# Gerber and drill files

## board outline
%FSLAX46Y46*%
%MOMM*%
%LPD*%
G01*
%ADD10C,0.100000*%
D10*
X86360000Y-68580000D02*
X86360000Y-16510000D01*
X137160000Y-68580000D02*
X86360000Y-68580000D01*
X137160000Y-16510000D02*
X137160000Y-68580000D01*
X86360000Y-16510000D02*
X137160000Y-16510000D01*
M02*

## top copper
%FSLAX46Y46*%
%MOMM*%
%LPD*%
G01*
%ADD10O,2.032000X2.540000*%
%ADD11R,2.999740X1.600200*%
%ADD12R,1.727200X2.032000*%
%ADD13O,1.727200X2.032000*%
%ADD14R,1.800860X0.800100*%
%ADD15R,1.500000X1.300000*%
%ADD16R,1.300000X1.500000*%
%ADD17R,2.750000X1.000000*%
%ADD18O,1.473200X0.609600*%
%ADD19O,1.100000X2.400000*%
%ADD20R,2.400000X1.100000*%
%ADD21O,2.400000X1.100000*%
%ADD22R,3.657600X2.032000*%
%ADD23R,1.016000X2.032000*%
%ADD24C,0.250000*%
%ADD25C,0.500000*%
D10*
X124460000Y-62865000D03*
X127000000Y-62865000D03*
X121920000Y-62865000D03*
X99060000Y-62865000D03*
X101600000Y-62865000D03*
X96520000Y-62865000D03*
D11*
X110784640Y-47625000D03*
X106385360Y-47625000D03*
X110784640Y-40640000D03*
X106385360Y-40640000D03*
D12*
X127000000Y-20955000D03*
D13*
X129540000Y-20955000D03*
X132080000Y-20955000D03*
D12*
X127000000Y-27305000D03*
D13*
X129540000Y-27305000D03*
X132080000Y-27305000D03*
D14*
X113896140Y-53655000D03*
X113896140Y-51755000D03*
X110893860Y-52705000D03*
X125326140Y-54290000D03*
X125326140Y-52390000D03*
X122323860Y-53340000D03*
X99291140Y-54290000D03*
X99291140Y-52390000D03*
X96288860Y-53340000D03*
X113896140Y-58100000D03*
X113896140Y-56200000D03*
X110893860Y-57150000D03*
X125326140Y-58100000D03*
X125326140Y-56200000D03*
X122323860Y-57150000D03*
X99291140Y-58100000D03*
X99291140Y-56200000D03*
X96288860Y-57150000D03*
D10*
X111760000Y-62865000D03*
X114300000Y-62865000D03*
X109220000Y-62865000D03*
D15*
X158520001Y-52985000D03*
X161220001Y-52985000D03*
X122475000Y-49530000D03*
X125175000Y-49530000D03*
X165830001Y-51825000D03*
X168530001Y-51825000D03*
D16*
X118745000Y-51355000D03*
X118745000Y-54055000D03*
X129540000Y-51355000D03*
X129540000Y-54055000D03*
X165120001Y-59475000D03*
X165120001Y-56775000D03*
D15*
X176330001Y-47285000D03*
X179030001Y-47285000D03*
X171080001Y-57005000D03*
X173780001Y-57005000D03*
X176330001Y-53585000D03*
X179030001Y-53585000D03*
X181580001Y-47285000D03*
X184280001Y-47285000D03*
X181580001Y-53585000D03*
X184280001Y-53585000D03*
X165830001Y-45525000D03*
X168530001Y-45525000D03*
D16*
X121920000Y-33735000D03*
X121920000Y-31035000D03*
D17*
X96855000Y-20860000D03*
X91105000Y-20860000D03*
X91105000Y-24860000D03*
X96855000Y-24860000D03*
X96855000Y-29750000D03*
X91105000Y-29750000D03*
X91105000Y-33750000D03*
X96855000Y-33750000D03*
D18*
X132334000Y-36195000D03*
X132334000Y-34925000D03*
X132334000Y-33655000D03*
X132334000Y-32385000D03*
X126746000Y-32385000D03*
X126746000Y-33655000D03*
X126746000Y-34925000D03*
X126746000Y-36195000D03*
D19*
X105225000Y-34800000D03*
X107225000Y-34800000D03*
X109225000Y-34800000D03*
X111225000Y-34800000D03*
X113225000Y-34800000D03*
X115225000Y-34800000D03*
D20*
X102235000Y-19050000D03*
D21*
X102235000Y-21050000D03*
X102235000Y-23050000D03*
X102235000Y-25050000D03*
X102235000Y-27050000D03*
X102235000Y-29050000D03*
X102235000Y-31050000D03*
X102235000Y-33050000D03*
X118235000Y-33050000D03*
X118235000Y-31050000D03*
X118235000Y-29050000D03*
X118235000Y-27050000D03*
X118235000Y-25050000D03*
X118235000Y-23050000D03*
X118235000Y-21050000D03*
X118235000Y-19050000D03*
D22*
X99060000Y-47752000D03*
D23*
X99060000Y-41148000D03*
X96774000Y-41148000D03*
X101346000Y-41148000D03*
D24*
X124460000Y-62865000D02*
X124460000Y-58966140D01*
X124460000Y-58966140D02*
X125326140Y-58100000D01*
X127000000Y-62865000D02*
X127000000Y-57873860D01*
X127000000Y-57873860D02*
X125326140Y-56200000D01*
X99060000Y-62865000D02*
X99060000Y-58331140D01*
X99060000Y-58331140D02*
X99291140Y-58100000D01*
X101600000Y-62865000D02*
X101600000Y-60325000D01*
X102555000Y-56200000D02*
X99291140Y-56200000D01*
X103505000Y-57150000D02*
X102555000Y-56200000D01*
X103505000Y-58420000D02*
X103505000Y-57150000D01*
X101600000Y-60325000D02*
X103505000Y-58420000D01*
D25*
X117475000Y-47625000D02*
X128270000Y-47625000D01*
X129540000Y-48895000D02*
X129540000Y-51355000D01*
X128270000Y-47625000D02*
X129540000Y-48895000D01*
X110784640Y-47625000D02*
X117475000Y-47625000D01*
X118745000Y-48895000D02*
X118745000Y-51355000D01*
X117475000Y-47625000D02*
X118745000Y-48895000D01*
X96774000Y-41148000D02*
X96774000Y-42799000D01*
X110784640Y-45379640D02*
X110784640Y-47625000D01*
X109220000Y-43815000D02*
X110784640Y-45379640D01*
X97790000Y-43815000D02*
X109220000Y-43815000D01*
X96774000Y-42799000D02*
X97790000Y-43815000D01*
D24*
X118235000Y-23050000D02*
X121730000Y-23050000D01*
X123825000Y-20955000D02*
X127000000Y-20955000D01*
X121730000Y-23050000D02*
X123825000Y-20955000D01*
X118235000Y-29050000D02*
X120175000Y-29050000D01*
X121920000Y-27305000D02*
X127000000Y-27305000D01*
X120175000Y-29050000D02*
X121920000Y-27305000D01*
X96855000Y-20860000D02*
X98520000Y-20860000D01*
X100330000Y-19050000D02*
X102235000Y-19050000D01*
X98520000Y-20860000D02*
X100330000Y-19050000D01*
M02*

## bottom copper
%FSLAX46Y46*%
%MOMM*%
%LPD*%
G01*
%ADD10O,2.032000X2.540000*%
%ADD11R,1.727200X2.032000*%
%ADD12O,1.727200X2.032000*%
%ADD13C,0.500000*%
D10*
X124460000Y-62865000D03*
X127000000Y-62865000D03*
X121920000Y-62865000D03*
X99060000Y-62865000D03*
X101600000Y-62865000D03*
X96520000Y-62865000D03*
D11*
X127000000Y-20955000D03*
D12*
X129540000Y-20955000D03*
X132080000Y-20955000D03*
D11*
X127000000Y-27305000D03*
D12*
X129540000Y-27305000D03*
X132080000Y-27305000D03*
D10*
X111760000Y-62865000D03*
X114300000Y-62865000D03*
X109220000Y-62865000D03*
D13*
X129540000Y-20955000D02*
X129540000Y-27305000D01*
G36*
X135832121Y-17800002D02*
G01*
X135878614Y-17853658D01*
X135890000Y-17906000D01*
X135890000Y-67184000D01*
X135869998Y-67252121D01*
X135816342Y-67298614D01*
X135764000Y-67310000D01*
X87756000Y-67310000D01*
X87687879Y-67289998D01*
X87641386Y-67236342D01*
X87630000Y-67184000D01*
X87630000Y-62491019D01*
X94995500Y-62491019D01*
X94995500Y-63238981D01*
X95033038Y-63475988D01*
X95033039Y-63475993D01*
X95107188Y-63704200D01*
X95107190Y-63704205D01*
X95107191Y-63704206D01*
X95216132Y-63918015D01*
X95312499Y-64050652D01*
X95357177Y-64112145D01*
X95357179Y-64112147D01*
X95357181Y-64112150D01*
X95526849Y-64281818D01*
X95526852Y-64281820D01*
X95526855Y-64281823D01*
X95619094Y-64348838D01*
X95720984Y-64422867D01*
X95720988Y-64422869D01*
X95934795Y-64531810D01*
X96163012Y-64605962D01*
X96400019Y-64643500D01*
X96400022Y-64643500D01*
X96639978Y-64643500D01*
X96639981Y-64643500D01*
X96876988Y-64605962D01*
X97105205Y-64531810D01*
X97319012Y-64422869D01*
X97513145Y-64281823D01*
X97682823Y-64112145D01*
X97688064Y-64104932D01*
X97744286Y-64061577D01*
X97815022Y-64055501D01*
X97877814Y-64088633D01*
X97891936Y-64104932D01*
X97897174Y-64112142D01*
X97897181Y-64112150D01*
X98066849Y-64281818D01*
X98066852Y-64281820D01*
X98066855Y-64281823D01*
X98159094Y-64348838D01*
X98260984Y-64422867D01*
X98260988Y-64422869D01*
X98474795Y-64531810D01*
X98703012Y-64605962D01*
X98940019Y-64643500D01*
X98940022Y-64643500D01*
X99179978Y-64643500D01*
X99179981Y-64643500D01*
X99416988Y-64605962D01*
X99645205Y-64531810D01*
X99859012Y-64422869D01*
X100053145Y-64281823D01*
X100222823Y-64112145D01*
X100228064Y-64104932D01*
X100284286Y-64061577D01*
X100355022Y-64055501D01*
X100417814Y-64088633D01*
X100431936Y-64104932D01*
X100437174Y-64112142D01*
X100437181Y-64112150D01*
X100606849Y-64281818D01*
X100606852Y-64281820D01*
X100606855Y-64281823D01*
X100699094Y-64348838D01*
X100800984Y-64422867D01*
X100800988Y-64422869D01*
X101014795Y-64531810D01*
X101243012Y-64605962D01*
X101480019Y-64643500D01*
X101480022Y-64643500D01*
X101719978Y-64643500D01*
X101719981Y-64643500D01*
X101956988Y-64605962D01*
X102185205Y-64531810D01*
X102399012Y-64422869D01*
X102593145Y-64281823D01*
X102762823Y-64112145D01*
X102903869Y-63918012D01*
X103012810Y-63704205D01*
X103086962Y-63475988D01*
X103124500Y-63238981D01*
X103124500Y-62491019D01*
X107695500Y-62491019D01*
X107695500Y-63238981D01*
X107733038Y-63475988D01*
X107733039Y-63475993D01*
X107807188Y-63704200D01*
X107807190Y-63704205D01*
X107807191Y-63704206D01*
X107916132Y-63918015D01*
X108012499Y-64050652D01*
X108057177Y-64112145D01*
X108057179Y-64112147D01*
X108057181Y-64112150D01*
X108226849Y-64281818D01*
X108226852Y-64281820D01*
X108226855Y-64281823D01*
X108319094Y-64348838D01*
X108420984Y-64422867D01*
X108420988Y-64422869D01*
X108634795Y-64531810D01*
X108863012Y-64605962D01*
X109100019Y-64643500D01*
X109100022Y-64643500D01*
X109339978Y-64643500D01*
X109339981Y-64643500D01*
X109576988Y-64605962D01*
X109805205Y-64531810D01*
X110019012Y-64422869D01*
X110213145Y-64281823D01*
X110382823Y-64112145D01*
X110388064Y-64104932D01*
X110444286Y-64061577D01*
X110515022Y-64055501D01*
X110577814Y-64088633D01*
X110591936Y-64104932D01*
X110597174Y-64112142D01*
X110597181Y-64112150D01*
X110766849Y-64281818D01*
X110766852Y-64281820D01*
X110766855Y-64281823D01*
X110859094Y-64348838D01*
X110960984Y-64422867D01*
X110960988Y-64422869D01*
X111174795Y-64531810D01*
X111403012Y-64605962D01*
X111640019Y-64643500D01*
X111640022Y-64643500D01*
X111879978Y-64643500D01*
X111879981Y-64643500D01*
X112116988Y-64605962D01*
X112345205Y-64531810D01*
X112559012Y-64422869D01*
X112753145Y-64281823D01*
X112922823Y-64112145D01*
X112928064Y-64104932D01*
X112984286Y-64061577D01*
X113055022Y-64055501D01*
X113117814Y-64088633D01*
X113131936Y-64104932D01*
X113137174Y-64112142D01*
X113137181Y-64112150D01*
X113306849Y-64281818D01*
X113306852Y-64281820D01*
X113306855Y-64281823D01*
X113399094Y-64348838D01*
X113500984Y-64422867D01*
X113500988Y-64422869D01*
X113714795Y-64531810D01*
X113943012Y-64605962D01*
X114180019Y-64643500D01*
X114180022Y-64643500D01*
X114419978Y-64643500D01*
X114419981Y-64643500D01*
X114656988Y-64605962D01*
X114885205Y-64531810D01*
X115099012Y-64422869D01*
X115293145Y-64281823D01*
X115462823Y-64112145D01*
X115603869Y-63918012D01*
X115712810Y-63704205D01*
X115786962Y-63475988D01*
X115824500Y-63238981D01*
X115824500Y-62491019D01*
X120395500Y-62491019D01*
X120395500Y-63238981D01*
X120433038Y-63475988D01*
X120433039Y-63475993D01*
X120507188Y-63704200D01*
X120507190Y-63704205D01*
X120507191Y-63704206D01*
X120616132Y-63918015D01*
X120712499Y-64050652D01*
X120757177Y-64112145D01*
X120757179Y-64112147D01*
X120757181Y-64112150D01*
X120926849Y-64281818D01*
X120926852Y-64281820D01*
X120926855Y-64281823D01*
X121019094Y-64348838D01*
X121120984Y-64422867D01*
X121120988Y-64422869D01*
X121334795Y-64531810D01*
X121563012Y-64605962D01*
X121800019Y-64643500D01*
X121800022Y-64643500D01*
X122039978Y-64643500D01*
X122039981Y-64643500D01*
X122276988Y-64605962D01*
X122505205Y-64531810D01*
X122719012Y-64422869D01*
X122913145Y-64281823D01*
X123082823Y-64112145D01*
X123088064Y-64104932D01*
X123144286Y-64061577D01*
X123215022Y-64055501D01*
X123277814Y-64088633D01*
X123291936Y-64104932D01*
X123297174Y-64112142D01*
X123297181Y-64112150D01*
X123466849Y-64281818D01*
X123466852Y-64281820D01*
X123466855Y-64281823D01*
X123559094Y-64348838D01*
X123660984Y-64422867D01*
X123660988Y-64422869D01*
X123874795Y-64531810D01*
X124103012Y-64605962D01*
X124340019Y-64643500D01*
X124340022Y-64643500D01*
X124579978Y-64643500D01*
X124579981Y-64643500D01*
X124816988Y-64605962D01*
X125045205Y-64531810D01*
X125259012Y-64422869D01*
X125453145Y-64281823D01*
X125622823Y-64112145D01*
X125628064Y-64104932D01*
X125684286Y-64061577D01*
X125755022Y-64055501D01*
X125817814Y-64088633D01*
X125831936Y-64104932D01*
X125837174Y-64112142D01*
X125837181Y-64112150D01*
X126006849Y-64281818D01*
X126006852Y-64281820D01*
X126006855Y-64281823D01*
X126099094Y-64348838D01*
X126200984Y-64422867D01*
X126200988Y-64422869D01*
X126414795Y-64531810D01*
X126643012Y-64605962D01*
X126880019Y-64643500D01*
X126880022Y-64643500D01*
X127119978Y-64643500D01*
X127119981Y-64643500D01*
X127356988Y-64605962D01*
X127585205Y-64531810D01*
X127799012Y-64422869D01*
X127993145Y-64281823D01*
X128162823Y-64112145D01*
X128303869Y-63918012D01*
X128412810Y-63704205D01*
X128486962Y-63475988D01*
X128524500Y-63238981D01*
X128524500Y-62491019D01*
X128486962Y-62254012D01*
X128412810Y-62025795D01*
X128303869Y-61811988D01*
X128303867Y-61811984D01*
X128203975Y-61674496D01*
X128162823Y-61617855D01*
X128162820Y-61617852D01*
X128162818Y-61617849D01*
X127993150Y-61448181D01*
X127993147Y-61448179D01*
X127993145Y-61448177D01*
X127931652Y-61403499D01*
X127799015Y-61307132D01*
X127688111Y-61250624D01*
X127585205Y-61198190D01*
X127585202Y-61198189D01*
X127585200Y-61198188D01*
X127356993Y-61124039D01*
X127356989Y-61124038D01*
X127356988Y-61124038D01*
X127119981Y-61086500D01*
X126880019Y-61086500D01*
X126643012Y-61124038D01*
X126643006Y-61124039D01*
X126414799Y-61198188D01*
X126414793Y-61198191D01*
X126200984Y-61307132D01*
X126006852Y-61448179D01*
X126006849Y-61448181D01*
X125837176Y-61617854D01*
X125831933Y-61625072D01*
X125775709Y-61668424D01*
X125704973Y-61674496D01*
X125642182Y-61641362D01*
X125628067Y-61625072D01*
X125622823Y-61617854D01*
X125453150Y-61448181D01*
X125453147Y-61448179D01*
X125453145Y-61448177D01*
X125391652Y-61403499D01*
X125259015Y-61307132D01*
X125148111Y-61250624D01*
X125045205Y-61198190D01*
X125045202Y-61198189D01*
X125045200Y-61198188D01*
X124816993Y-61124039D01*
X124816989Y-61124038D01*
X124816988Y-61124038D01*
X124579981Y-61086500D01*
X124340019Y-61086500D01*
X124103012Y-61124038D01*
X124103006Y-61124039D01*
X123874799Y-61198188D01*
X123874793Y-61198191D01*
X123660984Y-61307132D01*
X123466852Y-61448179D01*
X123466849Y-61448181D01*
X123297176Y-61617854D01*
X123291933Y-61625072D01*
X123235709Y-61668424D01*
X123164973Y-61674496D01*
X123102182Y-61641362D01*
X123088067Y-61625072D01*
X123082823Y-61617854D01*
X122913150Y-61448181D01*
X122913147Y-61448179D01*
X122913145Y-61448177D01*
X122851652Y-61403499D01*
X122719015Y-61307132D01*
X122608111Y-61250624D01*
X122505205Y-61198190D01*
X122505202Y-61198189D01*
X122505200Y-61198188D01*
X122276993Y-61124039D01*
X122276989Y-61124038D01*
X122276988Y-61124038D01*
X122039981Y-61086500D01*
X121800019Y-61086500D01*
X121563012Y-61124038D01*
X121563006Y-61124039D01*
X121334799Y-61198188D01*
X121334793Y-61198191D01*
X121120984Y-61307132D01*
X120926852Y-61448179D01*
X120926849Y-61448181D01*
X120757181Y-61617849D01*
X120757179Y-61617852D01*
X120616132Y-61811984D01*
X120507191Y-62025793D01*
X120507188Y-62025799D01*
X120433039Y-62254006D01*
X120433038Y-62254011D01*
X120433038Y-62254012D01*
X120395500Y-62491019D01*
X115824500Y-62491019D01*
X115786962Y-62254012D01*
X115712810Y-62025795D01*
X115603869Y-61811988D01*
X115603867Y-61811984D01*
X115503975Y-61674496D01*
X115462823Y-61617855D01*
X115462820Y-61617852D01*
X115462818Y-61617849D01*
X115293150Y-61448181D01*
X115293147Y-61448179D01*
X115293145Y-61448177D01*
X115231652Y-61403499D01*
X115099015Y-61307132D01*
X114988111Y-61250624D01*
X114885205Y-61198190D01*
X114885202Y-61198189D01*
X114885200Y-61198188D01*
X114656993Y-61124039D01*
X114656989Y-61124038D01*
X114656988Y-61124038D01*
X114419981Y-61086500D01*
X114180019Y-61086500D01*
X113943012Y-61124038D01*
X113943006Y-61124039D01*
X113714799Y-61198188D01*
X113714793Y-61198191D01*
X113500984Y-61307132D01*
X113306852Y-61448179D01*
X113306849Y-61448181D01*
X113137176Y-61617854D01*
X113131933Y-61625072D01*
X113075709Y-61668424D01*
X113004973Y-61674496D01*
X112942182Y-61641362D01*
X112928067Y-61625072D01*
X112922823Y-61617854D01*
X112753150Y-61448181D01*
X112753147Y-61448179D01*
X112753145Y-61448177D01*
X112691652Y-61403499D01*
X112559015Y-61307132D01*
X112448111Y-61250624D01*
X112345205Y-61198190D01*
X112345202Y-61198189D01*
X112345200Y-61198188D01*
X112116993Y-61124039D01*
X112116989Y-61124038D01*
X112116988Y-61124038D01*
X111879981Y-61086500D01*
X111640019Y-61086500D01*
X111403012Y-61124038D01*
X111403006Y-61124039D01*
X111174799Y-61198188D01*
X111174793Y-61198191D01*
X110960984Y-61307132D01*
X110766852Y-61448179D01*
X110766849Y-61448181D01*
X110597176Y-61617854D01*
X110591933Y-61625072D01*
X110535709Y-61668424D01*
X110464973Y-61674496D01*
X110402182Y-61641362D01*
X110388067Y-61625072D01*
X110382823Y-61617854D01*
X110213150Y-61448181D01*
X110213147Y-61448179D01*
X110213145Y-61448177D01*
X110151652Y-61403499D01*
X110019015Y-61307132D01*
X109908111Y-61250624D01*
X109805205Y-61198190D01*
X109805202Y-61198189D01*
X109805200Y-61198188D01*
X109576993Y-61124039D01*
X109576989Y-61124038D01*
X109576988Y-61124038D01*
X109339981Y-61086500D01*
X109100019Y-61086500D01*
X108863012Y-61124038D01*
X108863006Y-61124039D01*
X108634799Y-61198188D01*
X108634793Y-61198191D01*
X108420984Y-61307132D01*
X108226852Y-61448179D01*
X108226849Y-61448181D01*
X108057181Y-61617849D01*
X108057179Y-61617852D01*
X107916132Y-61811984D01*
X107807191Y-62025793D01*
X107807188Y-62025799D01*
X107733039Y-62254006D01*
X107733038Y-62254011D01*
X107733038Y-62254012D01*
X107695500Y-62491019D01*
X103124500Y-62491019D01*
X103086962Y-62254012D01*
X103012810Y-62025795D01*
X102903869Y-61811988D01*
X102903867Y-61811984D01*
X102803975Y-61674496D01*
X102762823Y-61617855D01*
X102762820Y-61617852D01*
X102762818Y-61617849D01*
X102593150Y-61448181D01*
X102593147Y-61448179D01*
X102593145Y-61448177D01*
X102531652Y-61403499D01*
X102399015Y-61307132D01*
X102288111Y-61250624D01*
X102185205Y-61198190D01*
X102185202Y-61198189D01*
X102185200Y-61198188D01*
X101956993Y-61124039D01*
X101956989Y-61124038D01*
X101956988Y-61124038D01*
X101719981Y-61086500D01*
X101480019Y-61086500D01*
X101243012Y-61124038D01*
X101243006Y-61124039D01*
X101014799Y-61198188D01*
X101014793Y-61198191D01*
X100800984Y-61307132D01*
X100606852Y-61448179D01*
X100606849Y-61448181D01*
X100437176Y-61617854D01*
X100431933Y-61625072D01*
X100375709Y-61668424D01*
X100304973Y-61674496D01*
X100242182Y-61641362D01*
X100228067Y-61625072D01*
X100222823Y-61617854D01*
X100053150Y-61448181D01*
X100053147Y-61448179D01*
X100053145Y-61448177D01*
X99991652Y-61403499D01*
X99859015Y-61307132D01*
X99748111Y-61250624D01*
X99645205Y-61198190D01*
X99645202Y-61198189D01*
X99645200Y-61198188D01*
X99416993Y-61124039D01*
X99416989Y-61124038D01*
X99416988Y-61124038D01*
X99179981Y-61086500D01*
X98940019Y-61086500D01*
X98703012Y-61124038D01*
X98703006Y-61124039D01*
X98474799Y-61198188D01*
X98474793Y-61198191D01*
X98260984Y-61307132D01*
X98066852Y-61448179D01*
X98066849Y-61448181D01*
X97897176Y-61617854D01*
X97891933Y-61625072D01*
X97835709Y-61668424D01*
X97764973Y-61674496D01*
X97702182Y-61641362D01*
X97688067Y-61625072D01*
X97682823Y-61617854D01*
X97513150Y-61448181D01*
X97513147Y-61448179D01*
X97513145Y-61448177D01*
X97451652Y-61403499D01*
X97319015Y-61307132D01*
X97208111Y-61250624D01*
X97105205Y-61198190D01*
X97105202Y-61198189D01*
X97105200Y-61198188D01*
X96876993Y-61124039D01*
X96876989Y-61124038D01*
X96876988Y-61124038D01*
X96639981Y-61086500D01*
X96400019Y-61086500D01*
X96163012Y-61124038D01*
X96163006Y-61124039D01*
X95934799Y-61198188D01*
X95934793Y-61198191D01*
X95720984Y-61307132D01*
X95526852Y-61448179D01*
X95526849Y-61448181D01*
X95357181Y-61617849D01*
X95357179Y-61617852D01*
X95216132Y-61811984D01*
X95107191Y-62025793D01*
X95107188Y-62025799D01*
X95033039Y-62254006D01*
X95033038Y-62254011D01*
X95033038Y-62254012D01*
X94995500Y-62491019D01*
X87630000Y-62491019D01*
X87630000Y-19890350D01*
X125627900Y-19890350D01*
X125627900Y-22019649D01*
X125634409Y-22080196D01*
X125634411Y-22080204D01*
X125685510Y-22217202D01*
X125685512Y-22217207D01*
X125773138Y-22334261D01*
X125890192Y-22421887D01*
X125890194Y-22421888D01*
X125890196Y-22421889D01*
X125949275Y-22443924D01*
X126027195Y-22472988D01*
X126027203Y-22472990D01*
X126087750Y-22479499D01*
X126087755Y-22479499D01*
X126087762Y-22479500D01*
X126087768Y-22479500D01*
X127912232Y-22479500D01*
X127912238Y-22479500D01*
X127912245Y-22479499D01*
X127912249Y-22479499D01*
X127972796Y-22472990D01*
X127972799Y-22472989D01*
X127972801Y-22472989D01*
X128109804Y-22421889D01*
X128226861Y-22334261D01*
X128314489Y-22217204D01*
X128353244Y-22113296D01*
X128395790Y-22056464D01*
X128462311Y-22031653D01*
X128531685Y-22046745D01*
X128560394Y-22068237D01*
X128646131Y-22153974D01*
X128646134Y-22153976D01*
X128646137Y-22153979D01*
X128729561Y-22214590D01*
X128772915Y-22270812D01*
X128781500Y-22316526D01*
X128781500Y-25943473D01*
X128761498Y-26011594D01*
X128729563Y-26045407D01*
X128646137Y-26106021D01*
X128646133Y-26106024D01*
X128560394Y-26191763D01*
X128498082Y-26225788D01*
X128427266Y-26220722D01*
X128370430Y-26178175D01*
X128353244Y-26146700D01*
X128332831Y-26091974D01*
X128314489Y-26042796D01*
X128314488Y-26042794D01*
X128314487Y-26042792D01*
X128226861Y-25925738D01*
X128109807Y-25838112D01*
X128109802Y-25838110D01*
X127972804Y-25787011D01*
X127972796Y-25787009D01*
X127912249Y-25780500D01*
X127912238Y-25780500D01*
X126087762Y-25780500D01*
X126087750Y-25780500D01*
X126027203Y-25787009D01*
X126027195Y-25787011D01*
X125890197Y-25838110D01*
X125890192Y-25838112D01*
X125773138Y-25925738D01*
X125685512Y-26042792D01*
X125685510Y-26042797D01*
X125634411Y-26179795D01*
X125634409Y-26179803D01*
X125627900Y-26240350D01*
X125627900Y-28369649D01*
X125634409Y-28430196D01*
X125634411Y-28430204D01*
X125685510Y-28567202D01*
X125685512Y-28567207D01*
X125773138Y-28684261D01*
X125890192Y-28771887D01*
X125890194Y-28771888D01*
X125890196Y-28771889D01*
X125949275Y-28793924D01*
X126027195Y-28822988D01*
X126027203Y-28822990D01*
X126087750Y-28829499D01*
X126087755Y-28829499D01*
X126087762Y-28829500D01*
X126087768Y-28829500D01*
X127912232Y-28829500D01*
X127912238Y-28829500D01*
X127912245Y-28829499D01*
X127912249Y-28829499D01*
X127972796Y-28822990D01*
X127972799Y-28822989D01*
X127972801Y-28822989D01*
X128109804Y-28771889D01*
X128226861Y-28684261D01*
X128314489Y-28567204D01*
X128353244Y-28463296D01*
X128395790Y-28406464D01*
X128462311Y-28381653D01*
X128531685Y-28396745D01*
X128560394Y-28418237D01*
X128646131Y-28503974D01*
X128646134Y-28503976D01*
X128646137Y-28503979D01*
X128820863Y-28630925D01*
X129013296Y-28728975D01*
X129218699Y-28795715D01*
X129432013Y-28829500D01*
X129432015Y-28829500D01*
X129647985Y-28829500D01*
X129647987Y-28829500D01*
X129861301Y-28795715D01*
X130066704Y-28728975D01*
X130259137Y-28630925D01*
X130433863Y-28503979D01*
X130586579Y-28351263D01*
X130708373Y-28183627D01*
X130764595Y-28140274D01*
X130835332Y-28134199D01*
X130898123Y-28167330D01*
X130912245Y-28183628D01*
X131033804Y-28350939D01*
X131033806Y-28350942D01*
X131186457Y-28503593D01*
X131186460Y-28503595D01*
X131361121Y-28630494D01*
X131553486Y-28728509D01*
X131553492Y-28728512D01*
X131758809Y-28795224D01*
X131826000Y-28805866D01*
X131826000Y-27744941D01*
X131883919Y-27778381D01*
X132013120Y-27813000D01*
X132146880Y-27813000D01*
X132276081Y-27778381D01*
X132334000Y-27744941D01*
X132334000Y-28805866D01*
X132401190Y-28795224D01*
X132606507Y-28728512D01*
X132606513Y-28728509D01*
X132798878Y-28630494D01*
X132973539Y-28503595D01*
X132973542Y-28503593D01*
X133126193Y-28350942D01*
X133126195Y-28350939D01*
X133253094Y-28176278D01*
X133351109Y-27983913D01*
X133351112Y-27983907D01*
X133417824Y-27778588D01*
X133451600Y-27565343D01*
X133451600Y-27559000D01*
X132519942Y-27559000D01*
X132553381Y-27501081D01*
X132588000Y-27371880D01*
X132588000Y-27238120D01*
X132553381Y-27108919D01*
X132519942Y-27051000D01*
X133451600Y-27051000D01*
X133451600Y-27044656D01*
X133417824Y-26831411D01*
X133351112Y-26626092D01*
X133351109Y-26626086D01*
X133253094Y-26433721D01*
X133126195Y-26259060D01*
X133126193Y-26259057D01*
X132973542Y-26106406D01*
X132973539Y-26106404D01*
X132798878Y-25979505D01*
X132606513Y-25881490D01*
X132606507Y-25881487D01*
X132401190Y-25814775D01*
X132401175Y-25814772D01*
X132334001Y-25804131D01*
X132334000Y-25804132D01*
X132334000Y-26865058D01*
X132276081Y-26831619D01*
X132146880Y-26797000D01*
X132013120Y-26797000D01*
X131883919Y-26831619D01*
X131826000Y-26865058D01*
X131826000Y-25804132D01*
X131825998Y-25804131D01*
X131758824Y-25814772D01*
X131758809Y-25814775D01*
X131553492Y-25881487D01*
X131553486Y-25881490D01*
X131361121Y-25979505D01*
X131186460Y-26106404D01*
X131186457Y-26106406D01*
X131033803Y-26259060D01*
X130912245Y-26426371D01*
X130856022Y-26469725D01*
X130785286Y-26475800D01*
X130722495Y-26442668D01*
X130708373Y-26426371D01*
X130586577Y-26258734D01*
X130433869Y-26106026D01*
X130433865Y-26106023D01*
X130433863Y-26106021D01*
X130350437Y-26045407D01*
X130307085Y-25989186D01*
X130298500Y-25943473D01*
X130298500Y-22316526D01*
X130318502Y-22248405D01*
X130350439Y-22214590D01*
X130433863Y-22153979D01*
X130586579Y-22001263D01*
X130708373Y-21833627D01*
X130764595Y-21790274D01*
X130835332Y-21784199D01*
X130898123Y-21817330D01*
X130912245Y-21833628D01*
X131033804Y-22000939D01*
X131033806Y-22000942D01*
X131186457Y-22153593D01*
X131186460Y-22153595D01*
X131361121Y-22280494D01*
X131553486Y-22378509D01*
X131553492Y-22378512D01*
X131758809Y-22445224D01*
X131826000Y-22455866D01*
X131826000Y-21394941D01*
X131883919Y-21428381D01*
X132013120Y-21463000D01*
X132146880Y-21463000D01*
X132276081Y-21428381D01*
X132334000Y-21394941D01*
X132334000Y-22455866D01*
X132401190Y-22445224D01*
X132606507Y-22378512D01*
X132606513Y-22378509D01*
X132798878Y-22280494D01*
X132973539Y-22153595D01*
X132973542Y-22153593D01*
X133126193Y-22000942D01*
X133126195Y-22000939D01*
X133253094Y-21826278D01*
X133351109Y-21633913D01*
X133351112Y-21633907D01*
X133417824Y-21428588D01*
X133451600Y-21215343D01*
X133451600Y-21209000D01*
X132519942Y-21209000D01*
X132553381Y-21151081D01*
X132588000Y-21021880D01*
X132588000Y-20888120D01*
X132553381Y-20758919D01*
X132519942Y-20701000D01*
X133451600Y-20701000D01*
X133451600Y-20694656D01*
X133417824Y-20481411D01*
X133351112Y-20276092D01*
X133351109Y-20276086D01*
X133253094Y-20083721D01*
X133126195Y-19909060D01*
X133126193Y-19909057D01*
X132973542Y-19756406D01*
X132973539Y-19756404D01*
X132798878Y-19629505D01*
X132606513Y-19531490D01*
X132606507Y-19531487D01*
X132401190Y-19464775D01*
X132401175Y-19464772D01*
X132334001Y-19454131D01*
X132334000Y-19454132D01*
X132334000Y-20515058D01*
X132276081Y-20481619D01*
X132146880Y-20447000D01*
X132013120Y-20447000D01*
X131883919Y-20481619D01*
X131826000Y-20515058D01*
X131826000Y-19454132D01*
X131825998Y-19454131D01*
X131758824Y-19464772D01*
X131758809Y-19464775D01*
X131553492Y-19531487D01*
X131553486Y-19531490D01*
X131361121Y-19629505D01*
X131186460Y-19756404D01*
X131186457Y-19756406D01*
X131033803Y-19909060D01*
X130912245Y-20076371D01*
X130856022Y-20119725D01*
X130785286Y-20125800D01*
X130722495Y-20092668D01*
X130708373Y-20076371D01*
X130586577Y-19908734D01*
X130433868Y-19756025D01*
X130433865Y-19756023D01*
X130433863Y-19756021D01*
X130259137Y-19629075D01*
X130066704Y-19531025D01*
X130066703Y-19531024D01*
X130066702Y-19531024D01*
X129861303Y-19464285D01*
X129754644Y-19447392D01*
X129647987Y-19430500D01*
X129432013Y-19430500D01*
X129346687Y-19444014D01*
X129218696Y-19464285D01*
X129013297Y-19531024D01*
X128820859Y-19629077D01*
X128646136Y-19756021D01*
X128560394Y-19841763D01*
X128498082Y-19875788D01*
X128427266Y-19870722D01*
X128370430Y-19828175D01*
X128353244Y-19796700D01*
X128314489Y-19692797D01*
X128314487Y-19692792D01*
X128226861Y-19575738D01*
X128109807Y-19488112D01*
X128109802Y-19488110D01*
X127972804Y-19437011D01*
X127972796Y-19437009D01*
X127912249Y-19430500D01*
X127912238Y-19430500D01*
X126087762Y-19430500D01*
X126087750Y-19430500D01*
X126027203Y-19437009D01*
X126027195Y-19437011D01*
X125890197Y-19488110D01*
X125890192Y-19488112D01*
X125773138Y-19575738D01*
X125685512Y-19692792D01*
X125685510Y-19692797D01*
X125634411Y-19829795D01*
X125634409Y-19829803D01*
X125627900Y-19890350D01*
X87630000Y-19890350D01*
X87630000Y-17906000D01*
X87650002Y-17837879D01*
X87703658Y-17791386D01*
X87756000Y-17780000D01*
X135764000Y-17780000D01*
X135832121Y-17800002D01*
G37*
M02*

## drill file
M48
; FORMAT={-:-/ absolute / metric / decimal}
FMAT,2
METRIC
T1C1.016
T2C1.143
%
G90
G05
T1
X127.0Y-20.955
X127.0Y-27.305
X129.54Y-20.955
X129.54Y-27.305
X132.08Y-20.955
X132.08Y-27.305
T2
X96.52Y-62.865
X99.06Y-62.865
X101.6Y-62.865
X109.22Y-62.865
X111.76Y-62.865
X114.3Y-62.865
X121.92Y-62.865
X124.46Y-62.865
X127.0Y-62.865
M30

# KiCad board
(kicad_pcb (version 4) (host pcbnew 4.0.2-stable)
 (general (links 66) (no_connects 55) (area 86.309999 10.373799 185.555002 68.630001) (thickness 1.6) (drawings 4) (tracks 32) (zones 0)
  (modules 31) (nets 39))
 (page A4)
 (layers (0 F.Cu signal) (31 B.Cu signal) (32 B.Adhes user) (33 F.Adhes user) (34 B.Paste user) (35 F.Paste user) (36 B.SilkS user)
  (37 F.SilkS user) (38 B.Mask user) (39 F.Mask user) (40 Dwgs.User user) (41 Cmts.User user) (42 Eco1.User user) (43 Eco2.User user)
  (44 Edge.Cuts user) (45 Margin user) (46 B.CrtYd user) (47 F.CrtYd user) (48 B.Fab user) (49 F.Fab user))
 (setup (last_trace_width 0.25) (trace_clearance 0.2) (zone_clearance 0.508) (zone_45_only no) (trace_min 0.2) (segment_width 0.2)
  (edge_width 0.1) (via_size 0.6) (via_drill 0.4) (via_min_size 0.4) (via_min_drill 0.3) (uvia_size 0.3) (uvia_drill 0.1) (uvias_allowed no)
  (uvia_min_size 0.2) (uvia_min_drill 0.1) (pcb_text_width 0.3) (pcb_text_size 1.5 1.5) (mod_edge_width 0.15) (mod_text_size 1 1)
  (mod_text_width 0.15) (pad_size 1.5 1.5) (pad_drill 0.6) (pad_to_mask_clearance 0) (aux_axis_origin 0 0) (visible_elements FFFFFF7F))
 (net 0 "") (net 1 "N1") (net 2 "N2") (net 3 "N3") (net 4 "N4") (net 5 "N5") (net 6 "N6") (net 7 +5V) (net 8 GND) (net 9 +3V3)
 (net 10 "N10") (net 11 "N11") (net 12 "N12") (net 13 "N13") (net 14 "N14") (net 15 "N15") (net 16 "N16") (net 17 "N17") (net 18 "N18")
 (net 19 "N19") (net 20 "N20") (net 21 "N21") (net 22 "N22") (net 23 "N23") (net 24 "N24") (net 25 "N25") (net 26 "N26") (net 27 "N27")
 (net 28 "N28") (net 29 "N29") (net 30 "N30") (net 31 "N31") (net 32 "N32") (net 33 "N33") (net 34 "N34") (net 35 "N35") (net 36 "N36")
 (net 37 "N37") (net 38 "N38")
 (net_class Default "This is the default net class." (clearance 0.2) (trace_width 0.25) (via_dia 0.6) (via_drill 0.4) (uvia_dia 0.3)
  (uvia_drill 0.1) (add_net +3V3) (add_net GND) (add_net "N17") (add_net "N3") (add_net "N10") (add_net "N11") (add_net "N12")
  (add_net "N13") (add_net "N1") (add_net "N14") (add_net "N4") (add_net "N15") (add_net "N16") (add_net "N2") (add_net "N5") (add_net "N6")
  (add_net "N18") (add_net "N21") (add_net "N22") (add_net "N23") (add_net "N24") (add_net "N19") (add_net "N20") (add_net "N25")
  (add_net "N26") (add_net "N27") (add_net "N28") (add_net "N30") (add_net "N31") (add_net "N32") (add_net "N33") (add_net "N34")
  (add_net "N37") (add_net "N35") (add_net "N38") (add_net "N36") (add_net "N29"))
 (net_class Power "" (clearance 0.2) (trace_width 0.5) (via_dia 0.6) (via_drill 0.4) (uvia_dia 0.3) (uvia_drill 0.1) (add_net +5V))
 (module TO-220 (layer F.Cu) (at 124.46 62.865)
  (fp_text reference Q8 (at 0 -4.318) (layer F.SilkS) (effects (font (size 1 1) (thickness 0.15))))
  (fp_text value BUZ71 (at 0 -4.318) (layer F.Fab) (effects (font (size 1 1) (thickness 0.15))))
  (pad 2 thru_hole oval (at 0 0) (size 2.032 2.54) (drill 1.143) (layers *.Cu *.Mask F.SilkS) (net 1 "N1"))
  (pad 3 thru_hole oval (at 2.54 0) (size 2.032 2.54) (drill 1.143) (layers *.Cu *.Mask F.SilkS) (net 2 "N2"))
  (pad 1 thru_hole oval (at -2.54 0) (size 2.032 2.54) (drill 1.143) (layers *.Cu *.Mask F.SilkS) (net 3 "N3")))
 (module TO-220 (layer F.Cu) (at 99.06 62.865)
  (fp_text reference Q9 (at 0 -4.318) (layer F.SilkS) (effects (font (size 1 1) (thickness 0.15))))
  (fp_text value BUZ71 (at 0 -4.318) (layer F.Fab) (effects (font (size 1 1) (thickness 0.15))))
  (pad 2 thru_hole oval (at 0 0) (size 2.032 2.54) (drill 1.143) (layers *.Cu *.Mask F.SilkS) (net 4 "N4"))
  (pad 3 thru_hole oval (at 2.54 0) (size 2.032 2.54) (drill 1.143) (layers *.Cu *.Mask F.SilkS) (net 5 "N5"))
  (pad 1 thru_hole oval (at -2.54 0) (size 2.032 2.54) (drill 1.143) (layers *.Cu *.Mask F.SilkS) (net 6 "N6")))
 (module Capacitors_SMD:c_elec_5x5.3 (layer F.Cu) (at 108.585 47.625)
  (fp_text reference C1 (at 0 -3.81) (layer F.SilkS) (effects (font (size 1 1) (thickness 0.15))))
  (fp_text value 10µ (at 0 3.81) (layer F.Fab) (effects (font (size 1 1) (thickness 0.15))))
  (pad 1 smd rect (at 2.19964 0) (size 2.99974 1.6002) (layers F.Cu F.Paste F.Mask) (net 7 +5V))
  (pad 2 smd rect (at -2.19964 0) (size 2.99974 1.6002) (layers F.Cu F.Paste F.Mask) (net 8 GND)))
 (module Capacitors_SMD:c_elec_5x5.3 (layer F.Cu) (at 108.585 40.64)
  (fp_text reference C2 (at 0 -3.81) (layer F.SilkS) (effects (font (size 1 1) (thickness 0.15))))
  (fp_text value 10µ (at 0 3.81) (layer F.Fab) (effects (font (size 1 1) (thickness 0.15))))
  (pad 1 smd rect (at 2.19964 0) (size 2.99974 1.6002) (layers F.Cu F.Paste F.Mask) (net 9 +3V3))
  (pad 2 smd rect (at -2.19964 0) (size 2.99974 1.6002) (layers F.Cu F.Paste F.Mask) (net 8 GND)))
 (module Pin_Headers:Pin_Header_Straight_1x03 (layer F.Cu) (at 127 20.955 90)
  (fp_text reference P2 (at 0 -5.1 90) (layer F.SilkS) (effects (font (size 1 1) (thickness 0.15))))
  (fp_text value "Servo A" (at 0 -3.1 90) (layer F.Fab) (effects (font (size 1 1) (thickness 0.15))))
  (pad 1 thru_hole rect (at 0 0 90) (size 2.032 1.7272) (drill 1.016) (layers *.Cu *.Mask F.SilkS) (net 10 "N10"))
  (pad 2 thru_hole oval (at 0 2.54 90) (size 2.032 1.7272) (drill 1.016) (layers *.Cu *.Mask F.SilkS) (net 7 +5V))
  (pad 3 thru_hole oval (at 0 5.08 90) (size 2.032 1.7272) (drill 1.016) (layers *.Cu *.Mask F.SilkS) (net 8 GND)))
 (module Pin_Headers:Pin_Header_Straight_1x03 (layer F.Cu) (at 127 27.305 90)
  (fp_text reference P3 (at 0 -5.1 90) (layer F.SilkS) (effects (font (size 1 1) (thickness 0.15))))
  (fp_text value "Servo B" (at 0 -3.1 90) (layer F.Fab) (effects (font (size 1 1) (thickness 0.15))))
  (pad 1 thru_hole rect (at 0 0 90) (size 2.032 1.7272) (drill 1.016) (layers *.Cu *.Mask F.SilkS) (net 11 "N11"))
  (pad 2 thru_hole oval (at 0 2.54 90) (size 2.032 1.7272) (drill 1.016) (layers *.Cu *.Mask F.SilkS) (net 7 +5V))
  (pad 3 thru_hole oval (at 0 5.08 90) (size 2.032 1.7272) (drill 1.016) (layers *.Cu *.Mask F.SilkS) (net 8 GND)))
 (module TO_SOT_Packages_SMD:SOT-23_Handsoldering (layer F.Cu) (at 112.395 52.705 90)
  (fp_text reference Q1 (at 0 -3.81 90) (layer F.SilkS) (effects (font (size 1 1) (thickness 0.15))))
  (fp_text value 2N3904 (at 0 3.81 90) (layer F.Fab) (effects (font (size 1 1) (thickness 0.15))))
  (pad 1 smd rect (at -0.95 1.50114 90) (size 0.8001 1.80086) (layers F.Cu F.Paste F.Mask) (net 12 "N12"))
  (pad 2 smd rect (at 0.95 1.50114 90) (size 0.8001 1.80086) (layers F.Cu F.Paste F.Mask) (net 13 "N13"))
  (pad 3 smd rect (at 0 -1.50114 90) (size 0.8001 1.80086) (layers F.Cu F.Paste F.Mask) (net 8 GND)))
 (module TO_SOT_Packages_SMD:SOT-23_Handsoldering (layer F.Cu) (at 123.825 53.34 90)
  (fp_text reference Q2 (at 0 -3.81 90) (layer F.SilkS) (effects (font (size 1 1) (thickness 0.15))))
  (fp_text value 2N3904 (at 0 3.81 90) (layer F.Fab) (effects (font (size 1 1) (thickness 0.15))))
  (pad 1 smd rect (at -0.95 1.50114 90) (size 0.8001 1.80086) (layers F.Cu F.Paste F.Mask) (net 1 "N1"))
  (pad 2 smd rect (at 0.95 1.50114 90) (size 0.8001 1.80086) (layers F.Cu F.Paste F.Mask) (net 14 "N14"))
  (pad 3 smd rect (at 0 -1.50114 90) (size 0.8001 1.80086) (layers F.Cu F.Paste F.Mask) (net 8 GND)))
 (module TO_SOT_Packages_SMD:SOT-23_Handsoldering (layer F.Cu) (at 97.79 53.34 90)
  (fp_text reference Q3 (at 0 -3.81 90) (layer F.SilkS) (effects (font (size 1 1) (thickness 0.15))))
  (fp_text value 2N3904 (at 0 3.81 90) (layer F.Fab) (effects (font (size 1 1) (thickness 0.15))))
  (pad 1 smd rect (at -0.95 1.50114 90) (size 0.8001 1.80086) (layers F.Cu F.Paste F.Mask) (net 4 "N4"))
  (pad 2 smd rect (at 0.95 1.50114 90) (size 0.8001 1.80086) (layers F.Cu F.Paste F.Mask) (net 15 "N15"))
  (pad 3 smd rect (at 0 -1.50114 90) (size 0.8001 1.80086) (layers F.Cu F.Paste F.Mask) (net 8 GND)))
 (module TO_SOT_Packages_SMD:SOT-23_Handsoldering (layer F.Cu) (at 112.395 57.15 90)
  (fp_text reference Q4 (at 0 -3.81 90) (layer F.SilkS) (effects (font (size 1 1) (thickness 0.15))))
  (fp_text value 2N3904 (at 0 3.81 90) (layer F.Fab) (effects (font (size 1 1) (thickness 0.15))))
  (pad 1 smd rect (at -0.95 1.50114 90) (size 0.8001 1.80086) (layers F.Cu F.Paste F.Mask) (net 12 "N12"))
  (pad 2 smd rect (at 0.95 1.50114 90) (size 0.8001 1.80086) (layers F.Cu F.Paste F.Mask) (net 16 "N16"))
  (pad 3 smd rect (at 0 -1.50114 90) (size 0.8001 1.80086) (layers F.Cu F.Paste F.Mask) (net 8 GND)))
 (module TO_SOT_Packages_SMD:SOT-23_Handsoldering (layer F.Cu) (at 123.825 57.15 90)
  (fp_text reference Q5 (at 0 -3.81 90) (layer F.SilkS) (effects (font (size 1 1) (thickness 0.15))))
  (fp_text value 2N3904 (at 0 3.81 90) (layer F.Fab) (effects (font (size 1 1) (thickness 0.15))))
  (pad 1 smd rect (at -0.95 1.50114 90) (size 0.8001 1.80086) (layers F.Cu F.Paste F.Mask) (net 1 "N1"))
  (pad 2 smd rect (at 0.95 1.50114 90) (size 0.8001 1.80086) (layers F.Cu F.Paste F.Mask) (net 2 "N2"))
  (pad 3 smd rect (at 0 -1.50114 90) (size 0.8001 1.80086) (layers F.Cu F.Paste F.Mask) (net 8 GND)))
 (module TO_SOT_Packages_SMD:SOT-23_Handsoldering (layer F.Cu) (at 97.79 57.15 90)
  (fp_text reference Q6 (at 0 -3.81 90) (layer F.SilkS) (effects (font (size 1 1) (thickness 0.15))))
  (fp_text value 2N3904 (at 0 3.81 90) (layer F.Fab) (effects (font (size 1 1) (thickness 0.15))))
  (pad 1 smd rect (at -0.95 1.50114 90) (size 0.8001 1.80086) (layers F.Cu F.Paste F.Mask) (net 4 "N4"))
  (pad 2 smd rect (at 0.95 1.50114 90) (size 0.8001 1.80086) (layers F.Cu F.Paste F.Mask) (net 5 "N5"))
  (pad 3 smd rect (at 0 -1.50114 90) (size 0.8001 1.80086) (layers F.Cu F.Paste F.Mask) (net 8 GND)))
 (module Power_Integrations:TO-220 (layer F.Cu) (at 111.76 62.865)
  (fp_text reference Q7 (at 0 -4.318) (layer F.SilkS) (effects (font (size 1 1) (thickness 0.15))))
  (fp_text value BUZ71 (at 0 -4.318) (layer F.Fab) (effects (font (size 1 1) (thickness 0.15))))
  (pad 2 thru_hole oval (at 0 0) (size 2.032 2.54) (drill 1.143) (layers *.Cu *.Mask F.SilkS) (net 12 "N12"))
  (pad 3 thru_hole oval (at 2.54 0) (size 2.032 2.54) (drill 1.143) (layers *.Cu *.Mask F.SilkS) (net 16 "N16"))
  (pad 1 thru_hole oval (at -2.54 0) (size 2.032 2.54) (drill 1.143) (layers *.Cu *.Mask F.SilkS) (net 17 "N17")))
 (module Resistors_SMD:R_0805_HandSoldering (layer F.Cu) (at 159.870001 52.985)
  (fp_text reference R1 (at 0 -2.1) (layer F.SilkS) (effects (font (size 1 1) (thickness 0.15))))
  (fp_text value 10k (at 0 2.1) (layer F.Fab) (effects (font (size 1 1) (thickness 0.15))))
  (pad 1 smd rect (at -1.35 0) (size 1.5 1.3) (layers F.Cu F.Paste F.Mask) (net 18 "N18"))
  (pad 2 smd rect (at 1.35 0) (size 1.5 1.3) (layers F.Cu F.Paste F.Mask) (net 13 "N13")))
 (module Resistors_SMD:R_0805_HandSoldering (layer F.Cu) (at 123.825 49.53)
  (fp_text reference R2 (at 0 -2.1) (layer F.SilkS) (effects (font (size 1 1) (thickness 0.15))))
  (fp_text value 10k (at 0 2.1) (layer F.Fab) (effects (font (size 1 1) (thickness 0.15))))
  (pad 1 smd rect (at -1.35 0) (size 1.5 1.3) (layers F.Cu F.Paste F.Mask) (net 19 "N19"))
  (pad 2 smd rect (at 1.35 0) (size 1.5 1.3) (layers F.Cu F.Paste F.Mask) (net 14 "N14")))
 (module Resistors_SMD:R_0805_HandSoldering (layer F.Cu) (at 167.180001 51.825)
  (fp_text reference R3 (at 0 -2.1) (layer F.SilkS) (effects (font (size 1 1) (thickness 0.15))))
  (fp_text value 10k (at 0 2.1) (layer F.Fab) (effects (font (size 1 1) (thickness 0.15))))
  (pad 1 smd rect (at -1.35 0) (size 1.5 1.3) (layers F.Cu F.Paste F.Mask) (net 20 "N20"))
  (pad 2 smd rect (at 1.35 0) (size 1.5 1.3) (layers F.Cu F.Paste F.Mask) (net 15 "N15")))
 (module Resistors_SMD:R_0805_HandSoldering (layer F.Cu) (at 118.745 52.705 270)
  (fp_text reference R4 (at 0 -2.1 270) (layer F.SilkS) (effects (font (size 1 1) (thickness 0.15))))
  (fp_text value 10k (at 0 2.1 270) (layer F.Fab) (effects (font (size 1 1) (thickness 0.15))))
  (pad 1 smd rect (at -1.35 0 270) (size 1.5 1.3) (layers F.Cu F.Paste F.Mask) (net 7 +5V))
  (pad 2 smd rect (at 1.35 0 270) (size 1.5 1.3) (layers F.Cu F.Paste F.Mask) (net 12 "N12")))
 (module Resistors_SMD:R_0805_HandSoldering (layer F.Cu) (at 129.54 52.705 270)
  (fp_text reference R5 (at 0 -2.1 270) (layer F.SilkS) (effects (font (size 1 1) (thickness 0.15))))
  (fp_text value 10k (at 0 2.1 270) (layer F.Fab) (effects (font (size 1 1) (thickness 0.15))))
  (pad 1 smd rect (at -1.35 0 270) (size 1.5 1.3) (layers F.Cu F.Paste F.Mask) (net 7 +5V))
  (pad 2 smd rect (at 1.35 0 270) (size 1.5 1.3) (layers F.Cu F.Paste F.Mask) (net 1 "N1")))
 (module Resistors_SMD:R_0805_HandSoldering (layer F.Cu) (at 165.120001 58.125 90)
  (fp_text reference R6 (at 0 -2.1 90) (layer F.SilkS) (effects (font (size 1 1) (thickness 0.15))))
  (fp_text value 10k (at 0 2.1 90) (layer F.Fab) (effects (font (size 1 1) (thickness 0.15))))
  (pad 1 smd rect (at -1.35 0 90) (size 1.5 1.3) (layers F.Cu F.Paste F.Mask) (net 7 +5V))
  (pad 2 smd rect (at 1.35 0 90) (size 1.5 1.3) (layers F.Cu F.Paste F.Mask) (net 4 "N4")))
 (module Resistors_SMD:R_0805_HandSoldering (layer F.Cu) (at 177.680001 47.285)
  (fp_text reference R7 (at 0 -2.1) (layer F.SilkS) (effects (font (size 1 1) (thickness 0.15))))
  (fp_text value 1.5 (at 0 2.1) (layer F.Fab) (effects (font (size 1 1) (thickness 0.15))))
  (pad 1 smd rect (at -1.35 0) (size 1.5 1.3) (layers F.Cu F.Paste F.Mask) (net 16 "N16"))
  (pad 2 smd rect (at 1.35 0) (size 1.5 1.3) (layers F.Cu F.Paste F.Mask) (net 8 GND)))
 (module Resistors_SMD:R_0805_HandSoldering (layer F.Cu) (at 172.430001 57.005)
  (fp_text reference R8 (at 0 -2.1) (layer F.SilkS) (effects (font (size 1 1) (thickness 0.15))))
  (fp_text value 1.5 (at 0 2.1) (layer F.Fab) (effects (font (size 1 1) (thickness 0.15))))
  (pad 1 smd rect (at -1.35 0) (size 1.5 1.3) (layers F.Cu F.Paste F.Mask) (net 2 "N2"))
  (pad 2 smd rect (at 1.35 0) (size 1.5 1.3) (layers F.Cu F.Paste F.Mask) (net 8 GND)))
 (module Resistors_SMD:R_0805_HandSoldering (layer F.Cu) (at 177.680001 53.585)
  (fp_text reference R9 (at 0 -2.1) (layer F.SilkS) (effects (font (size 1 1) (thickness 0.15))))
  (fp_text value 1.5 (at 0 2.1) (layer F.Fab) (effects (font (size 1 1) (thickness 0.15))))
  (pad 1 smd rect (at -1.35 0) (size 1.5 1.3) (layers F.Cu F.Paste F.Mask) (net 5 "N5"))
  (pad 2 smd rect (at 1.35 0) (size 1.5 1.3) (layers F.Cu F.Paste F.Mask) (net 8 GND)))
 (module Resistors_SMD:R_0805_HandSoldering (layer F.Cu) (at 182.930001 47.285)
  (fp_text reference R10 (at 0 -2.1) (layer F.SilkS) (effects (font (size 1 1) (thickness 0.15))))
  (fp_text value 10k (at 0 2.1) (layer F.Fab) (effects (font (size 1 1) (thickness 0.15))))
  (pad 1 smd rect (at -1.35 0) (size 1.5 1.3) (layers F.Cu F.Paste F.Mask) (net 9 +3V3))
  (pad 2 smd rect (at 1.35 0) (size 1.5 1.3) (layers F.Cu F.Paste F.Mask) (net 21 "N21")))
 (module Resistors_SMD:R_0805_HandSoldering (layer F.Cu) (at 182.930001 53.585)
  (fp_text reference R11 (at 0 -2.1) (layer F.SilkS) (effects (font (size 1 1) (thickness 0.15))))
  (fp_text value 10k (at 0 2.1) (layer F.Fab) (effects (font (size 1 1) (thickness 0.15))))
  (pad 1 smd rect (at -1.35 0) (size 1.5 1.3) (layers F.Cu F.Paste F.Mask) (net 9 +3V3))
  (pad 2 smd rect (at 1.35 0) (size 1.5 1.3) (layers F.Cu F.Paste F.Mask) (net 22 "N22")))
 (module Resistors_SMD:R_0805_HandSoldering (layer F.Cu) (at 167.180001 45.525)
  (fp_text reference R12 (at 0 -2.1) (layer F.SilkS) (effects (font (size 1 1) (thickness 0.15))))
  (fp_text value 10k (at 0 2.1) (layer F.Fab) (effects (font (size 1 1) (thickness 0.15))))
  (pad 1 smd rect (at -1.35 0) (size 1.5 1.3) (layers F.Cu F.Paste F.Mask) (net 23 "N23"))
  (pad 2 smd rect (at 1.35 0) (size 1.5 1.3) (layers F.Cu F.Paste F.Mask) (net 8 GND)))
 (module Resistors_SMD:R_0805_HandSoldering (layer F.Cu) (at 121.92 32.385 90)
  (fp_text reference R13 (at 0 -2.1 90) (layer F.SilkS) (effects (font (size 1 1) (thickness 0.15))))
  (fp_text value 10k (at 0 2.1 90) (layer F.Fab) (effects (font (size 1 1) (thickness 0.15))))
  (pad 1 smd rect (at -1.35 0 90) (size 1.5 1.3) (layers F.Cu F.Paste F.Mask) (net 9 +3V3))
  (pad 2 smd rect (at 1.35 0 90) (size 1.5 1.3) (layers F.Cu F.Paste F.Mask) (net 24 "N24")))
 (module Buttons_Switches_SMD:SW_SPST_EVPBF (layer F.Cu) (at 93.98 22.86)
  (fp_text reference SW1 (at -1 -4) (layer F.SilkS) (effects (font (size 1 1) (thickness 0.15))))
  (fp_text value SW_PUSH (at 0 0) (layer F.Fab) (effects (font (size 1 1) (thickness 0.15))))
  (pad 1 smd rect (at 2.875 -2) (size 2.75 1) (layers F.Cu F.Paste F.Mask) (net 21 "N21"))
  (pad 1 smd rect (at -2.875 -2) (size 2.75 1) (layers F.Cu F.Paste F.Mask) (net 21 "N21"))
  (pad 2 smd rect (at -2.875 2) (size 2.75 1) (layers F.Cu F.Paste F.Mask) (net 8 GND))
  (pad 2 smd rect (at 2.875 2) (size 2.75 1) (layers F.Cu F.Paste F.Mask) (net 8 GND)))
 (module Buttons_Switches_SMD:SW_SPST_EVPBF (layer F.Cu) (at 93.98 31.75)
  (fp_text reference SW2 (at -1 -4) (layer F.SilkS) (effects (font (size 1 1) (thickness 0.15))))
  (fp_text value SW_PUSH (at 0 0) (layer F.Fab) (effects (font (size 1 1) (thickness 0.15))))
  (pad 1 smd rect (at 2.875 -2) (size 2.75 1) (layers F.Cu F.Paste F.Mask) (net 24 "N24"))
  (pad 1 smd rect (at -2.875 -2) (size 2.75 1) (layers F.Cu F.Paste F.Mask) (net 24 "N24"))
  (pad 2 smd rect (at -2.875 2) (size 2.75 1) (layers F.Cu F.Paste F.Mask) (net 8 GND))
  (pad 2 smd rect (at 2.875 2) (size 2.75 1) (layers F.Cu F.Paste F.Mask) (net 8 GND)))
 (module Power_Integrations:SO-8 (layer F.Cu) (at 129.54 34.29 90)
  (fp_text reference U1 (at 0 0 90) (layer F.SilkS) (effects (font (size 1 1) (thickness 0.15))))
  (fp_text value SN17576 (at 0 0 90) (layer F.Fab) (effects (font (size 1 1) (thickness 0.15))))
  (pad 1 smd oval (at -1.905 2.794 90) (size 0.6096 1.4732) (layers F.Cu F.Paste F.Mask) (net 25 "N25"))
  (pad 2 smd oval (at -0.635 2.794 90) (size 0.6096 1.4732) (layers F.Cu F.Paste F.Mask) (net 8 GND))
  (pad 3 smd oval (at 0.635 2.794 90) (size 0.6096 1.4732) (layers F.Cu F.Paste F.Mask) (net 8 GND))
  (pad 4 smd oval (at 1.905 2.794 90) (size 0.6096 1.4732) (layers F.Cu F.Paste F.Mask) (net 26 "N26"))
  (pad 5 smd oval (at 1.905 -2.794 90) (size 0.6096 1.4732) (layers F.Cu F.Paste F.Mask) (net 8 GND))
  (pad 6 smd oval (at 0.635 -2.794 90) (size 0.6096 1.4732) (layers F.Cu F.Paste F.Mask) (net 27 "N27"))
  (pad 7 smd oval (at -0.635 -2.794 90) (size 0.6096 1.4732) (layers F.Cu F.Paste F.Mask) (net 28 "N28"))
  (pad 8 smd oval (at -1.905 -2.794 90) (size 0.6096 1.4732) (layers F.Cu F.Paste F.Mask) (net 9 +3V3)))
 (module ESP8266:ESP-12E (layer F.Cu) (at 102.235 19.05)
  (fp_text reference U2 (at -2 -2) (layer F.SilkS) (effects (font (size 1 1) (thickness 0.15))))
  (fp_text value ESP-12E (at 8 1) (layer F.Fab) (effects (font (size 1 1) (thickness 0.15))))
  (pad 9 smd oval (at 2.99 15.75 90) (size 2.4 1.1) (layers F.Cu F.Paste F.Mask) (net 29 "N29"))
  (pad 10 smd oval (at 4.99 15.75 90) (size 2.4 1.1) (layers F.Cu F.Paste F.Mask) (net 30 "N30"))
  (pad 11 smd oval (at 6.99 15.75 90) (size 2.4 1.1) (layers F.Cu F.Paste F.Mask) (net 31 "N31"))
  (pad 12 smd oval (at 8.99 15.75 90) (size 2.4 1.1) (layers F.Cu F.Paste F.Mask) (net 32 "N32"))
  (pad 13 smd oval (at 10.99 15.75 90) (size 2.4 1.1) (layers F.Cu F.Paste F.Mask) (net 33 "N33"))
  (pad 14 smd oval (at 12.99 15.75 90) (size 2.4 1.1) (layers F.Cu F.Paste F.Mask) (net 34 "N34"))
  (pad 1 smd rect (at 0 0) (size 2.4 1.1) (layers F.Cu F.Paste F.Mask) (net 21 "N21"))
  (pad 2 smd oval (at 0 2) (size 2.4 1.1) (layers F.Cu F.Paste F.Mask) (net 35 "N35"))
  (pad 3 smd oval (at 0 4) (size 2.4 1.1) (layers F.Cu F.Paste F.Mask) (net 22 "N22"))
  (pad 4 smd oval (at 0 6) (size 2.4 1.1) (layers F.Cu F.Paste F.Mask) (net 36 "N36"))
  (pad 5 smd oval (at 0 8) (size 2.4 1.1) (layers F.Cu F.Paste F.Mask) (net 18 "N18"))
  (pad 6 smd oval (at 0 10) (size 2.4 1.1) (layers F.Cu F.Paste F.Mask) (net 19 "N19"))
  (pad 7 smd oval (at 0 12) (size 2.4 1.1) (layers F.Cu F.Paste F.Mask) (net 20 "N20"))
  (pad 8 smd oval (at 0 14) (size 2.4 1.1) (layers F.Cu F.Paste F.Mask) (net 9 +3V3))
  (pad 15 smd oval (at 16 14) (size 2.4 1.1) (layers F.Cu F.Paste F.Mask) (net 8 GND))
  (pad 16 smd oval (at 16 12) (size 2.4 1.1) (layers F.Cu F.Paste F.Mask) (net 23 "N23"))
  (pad 17 smd oval (at 16 10) (size 2.4 1.1) (layers F.Cu F.Paste F.Mask) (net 11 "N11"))
  (pad 18 smd oval (at 16 8) (size 2.4 1.1) (layers F.Cu F.Paste F.Mask) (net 24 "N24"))
  (pad 19 smd oval (at 16 6) (size 2.4 1.1) (layers F.Cu F.Paste F.Mask) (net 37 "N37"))
  (pad 20 smd oval (at 16 4) (size 2.4 1.1) (layers F.Cu F.Paste F.Mask) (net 10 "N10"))
  (pad 21 smd oval (at 16 2) (size 2.4 1.1) (layers F.Cu F.Paste F.Mask) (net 25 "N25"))
  (pad 22 smd oval (at 16 0) (size 2.4 1.1) (layers F.Cu F.Paste F.Mask) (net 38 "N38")))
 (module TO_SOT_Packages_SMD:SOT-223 (layer F.Cu) (at 99.06 44.45 180)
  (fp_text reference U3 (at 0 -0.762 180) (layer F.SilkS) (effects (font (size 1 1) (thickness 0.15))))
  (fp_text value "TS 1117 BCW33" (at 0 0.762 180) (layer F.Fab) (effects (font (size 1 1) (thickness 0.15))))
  (pad 4 smd rect (at 0 -3.302 180) (size 3.6576 2.032) (layers F.Cu F.Paste F.Mask))
  (pad 2 smd rect (at 0 3.302 180) (size 1.016 2.032) (layers F.Cu F.Paste F.Mask) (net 8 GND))
  (pad 3 smd rect (at 2.286 3.302 180) (size 1.016 2.032) (layers F.Cu F.Paste F.Mask) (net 7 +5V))
  (pad 1 smd rect (at -2.286 3.302 180) (size 1.016 2.032) (layers F.Cu F.Paste F.Mask) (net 9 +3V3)))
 (gr_line (start 86.36 68.58) (end 86.36 16.51) (angle 90) (layer Edge.Cuts) (width 0.1))
 (gr_line (start 137.16 68.58) (end 86.36 68.58) (angle 90) (layer Edge.Cuts) (width 0.1))
 (gr_line (start 137.16 16.51) (end 137.16 68.58) (angle 90) (layer Edge.Cuts) (width 0.1))
 (gr_line (start 86.36 16.51) (end 137.16 16.51) (angle 90) (layer Edge.Cuts) (width 0.1))
 (segment (start 124.46 62.865) (end 124.46 58.96614) (width 0.25) (layer F.Cu) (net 1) (status 400000))
 (segment (start 124.46 58.96614) (end 125.32614 58.1) (width 0.25) (layer F.Cu) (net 1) (status 800000))
 (segment (start 127 62.865) (end 127 57.87386) (width 0.25) (layer F.Cu) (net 2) (status 400000))
 (segment (start 127 57.87386) (end 125.32614 56.2) (width 0.25) (layer F.Cu) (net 2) (status 800000))
 (segment (start 99.06 62.865) (end 99.06 58.33114) (width 0.25) (layer F.Cu) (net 4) (status C00000))
 (segment (start 99.06 58.33114) (end 99.29114 58.1) (width 0.25) (layer F.Cu) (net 4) (status C00000))
 (segment (start 101.6 62.865) (end 101.6 60.325) (width 0.25) (layer F.Cu) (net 5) (status 400000))
 (segment (start 102.555 56.2) (end 99.29114 56.2) (width 0.25) (layer F.Cu) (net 5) (status 800000))
 (segment (start 103.505 57.15) (end 102.555 56.2) (width 0.25) (layer F.Cu) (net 5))
 (segment (start 103.505 58.42) (end 103.505 57.15) (width 0.25) (layer F.Cu) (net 5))
 (segment (start 101.6 60.325) (end 103.505 58.42) (width 0.25) (layer F.Cu) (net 5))
 (segment (start 129.54 20.955) (end 129.54 27.305) (width 0.5) (layer B.Cu) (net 7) (status C00000))
 (segment (start 117.475 47.625) (end 128.27 47.625) (width 0.5) (layer F.Cu) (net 7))
 (segment (start 129.54 48.895) (end 129.54 51.355) (width 0.5) (layer F.Cu) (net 7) (status 800000))
 (segment (start 128.27 47.625) (end 129.54 48.895) (width 0.5) (layer F.Cu) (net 7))
 (segment (start 110.78464 47.625) (end 117.475 47.625) (width 0.5) (layer F.Cu) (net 7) (status 400000))
 (segment (start 118.745 48.895) (end 118.745 51.355) (width 0.5) (layer F.Cu) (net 7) (status 800000))
 (segment (start 117.475 47.625) (end 118.745 48.895) (width 0.5) (layer F.Cu) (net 7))
 (segment (start 96.774 41.148) (end 96.774 42.799) (width 0.5) (layer F.Cu) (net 7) (status 400000))
 (segment (start 110.78464 45.37964) (end 110.78464 47.625) (width 0.5) (layer F.Cu) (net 7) (status 800000))
 (segment (start 109.22 43.815) (end 110.78464 45.37964) (width 0.5) (layer F.Cu) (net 7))
 (segment (start 97.79 43.815) (end 109.22 43.815) (width 0.5) (layer F.Cu) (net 7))
 (segment (start 96.774 42.799) (end 97.79 43.815) (width 0.5) (layer F.Cu) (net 7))
 (segment (start 118.235 23.05) (end 121.73 23.05) (width 0.25) (layer F.Cu) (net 10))
 (segment (start 123.825 20.955) (end 127 20.955) (width 0.25) (layer F.Cu) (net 10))
 (segment (start 121.73 23.05) (end 123.825 20.955) (width 0.25) (layer F.Cu) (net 10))
 (segment (start 118.235 29.05) (end 120.175 29.05) (width 0.25) (layer F.Cu) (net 11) (status 400000))
 (segment (start 121.92 27.305) (end 127 27.305) (width 0.25) (layer F.Cu) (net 11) (status 800000))
 (segment (start 120.175 29.05) (end 121.92 27.305) (width 0.25) (layer F.Cu) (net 11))
 (segment (start 96.855 20.86) (end 98.52 20.86) (width 0.25) (layer F.Cu) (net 21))
 (segment (start 100.33 19.05) (end 102.235 19.05) (width 0.25) (layer F.Cu) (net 21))
 (segment (start 98.52 20.86) (end 100.33 19.05) (width 0.25) (layer F.Cu) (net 21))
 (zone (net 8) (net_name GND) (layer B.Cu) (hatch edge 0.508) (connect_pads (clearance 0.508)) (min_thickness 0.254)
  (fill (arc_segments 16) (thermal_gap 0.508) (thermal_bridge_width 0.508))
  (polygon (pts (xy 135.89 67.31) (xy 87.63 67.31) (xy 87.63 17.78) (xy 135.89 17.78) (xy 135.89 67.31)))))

